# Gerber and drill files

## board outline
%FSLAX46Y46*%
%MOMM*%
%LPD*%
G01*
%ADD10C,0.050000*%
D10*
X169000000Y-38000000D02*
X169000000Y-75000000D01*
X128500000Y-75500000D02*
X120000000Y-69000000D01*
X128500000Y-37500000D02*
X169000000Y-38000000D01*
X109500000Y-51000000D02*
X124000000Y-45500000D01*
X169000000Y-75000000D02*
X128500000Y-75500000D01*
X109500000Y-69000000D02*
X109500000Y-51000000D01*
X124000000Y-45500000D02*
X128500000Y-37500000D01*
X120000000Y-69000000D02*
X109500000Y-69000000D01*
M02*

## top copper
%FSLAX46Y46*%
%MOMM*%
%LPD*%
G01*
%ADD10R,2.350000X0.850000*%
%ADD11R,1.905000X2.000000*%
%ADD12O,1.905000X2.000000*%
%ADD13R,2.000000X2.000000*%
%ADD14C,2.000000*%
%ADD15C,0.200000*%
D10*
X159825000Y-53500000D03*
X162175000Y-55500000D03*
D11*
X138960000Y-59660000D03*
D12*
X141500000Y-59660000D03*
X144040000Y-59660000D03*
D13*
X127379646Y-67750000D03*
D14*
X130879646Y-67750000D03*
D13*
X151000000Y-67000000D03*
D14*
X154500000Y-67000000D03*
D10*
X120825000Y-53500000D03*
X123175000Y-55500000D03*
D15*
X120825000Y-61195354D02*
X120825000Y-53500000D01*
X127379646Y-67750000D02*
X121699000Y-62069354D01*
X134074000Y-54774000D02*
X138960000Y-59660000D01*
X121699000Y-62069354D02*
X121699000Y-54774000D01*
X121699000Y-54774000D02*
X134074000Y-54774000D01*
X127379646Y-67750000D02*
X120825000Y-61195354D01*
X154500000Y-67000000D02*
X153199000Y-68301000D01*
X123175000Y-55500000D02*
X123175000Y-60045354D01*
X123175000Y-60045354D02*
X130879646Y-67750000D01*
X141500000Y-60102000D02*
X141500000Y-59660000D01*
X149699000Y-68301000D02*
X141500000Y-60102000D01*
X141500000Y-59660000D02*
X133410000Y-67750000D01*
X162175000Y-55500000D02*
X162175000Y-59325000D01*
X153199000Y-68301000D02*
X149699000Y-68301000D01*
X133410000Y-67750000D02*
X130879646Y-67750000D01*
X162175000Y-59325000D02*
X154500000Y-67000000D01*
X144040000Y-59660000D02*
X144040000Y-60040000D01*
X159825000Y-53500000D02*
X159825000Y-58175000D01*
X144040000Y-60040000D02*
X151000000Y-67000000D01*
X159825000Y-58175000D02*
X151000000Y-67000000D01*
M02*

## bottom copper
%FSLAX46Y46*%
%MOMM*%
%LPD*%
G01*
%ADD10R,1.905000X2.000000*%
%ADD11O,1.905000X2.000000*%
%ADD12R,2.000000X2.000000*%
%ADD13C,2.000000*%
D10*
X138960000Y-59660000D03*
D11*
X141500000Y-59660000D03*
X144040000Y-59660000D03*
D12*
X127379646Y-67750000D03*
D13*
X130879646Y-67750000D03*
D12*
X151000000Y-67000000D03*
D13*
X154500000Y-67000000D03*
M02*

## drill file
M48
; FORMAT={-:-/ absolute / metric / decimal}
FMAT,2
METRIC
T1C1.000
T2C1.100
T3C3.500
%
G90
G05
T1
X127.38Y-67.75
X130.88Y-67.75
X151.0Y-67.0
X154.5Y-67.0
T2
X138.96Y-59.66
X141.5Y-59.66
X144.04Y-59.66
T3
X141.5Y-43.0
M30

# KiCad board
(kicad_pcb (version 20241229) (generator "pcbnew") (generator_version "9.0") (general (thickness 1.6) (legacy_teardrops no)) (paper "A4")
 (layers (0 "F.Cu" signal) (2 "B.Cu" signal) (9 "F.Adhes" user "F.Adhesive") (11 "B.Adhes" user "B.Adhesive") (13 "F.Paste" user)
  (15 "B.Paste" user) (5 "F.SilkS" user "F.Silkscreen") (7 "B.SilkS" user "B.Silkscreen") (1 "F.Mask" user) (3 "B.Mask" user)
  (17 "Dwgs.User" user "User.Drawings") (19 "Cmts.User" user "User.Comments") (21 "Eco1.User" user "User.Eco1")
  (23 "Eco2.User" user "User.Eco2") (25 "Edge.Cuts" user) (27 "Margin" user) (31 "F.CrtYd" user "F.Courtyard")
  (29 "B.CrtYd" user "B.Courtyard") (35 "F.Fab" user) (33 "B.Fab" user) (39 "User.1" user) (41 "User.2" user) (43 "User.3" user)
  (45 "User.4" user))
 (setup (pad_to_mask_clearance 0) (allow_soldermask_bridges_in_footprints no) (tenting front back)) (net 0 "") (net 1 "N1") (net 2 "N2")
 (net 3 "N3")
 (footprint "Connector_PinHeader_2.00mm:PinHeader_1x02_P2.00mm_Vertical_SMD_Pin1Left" (layer "F.Cu") (at 161 54.5)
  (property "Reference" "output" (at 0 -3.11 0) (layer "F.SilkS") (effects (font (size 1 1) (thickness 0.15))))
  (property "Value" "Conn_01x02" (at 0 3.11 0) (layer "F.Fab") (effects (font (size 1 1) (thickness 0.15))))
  (pad "1" smd rect (at -1.175 -1) (size 2.35 0.85) (layers "F.Cu" "F.Mask" "F.Paste") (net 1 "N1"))
  (pad "2" smd rect (at 1.175 1) (size 2.35 0.85) (layers "F.Cu" "F.Mask" "F.Paste") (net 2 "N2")))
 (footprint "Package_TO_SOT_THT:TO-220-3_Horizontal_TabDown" (layer "F.Cu") (at 138.96 59.66)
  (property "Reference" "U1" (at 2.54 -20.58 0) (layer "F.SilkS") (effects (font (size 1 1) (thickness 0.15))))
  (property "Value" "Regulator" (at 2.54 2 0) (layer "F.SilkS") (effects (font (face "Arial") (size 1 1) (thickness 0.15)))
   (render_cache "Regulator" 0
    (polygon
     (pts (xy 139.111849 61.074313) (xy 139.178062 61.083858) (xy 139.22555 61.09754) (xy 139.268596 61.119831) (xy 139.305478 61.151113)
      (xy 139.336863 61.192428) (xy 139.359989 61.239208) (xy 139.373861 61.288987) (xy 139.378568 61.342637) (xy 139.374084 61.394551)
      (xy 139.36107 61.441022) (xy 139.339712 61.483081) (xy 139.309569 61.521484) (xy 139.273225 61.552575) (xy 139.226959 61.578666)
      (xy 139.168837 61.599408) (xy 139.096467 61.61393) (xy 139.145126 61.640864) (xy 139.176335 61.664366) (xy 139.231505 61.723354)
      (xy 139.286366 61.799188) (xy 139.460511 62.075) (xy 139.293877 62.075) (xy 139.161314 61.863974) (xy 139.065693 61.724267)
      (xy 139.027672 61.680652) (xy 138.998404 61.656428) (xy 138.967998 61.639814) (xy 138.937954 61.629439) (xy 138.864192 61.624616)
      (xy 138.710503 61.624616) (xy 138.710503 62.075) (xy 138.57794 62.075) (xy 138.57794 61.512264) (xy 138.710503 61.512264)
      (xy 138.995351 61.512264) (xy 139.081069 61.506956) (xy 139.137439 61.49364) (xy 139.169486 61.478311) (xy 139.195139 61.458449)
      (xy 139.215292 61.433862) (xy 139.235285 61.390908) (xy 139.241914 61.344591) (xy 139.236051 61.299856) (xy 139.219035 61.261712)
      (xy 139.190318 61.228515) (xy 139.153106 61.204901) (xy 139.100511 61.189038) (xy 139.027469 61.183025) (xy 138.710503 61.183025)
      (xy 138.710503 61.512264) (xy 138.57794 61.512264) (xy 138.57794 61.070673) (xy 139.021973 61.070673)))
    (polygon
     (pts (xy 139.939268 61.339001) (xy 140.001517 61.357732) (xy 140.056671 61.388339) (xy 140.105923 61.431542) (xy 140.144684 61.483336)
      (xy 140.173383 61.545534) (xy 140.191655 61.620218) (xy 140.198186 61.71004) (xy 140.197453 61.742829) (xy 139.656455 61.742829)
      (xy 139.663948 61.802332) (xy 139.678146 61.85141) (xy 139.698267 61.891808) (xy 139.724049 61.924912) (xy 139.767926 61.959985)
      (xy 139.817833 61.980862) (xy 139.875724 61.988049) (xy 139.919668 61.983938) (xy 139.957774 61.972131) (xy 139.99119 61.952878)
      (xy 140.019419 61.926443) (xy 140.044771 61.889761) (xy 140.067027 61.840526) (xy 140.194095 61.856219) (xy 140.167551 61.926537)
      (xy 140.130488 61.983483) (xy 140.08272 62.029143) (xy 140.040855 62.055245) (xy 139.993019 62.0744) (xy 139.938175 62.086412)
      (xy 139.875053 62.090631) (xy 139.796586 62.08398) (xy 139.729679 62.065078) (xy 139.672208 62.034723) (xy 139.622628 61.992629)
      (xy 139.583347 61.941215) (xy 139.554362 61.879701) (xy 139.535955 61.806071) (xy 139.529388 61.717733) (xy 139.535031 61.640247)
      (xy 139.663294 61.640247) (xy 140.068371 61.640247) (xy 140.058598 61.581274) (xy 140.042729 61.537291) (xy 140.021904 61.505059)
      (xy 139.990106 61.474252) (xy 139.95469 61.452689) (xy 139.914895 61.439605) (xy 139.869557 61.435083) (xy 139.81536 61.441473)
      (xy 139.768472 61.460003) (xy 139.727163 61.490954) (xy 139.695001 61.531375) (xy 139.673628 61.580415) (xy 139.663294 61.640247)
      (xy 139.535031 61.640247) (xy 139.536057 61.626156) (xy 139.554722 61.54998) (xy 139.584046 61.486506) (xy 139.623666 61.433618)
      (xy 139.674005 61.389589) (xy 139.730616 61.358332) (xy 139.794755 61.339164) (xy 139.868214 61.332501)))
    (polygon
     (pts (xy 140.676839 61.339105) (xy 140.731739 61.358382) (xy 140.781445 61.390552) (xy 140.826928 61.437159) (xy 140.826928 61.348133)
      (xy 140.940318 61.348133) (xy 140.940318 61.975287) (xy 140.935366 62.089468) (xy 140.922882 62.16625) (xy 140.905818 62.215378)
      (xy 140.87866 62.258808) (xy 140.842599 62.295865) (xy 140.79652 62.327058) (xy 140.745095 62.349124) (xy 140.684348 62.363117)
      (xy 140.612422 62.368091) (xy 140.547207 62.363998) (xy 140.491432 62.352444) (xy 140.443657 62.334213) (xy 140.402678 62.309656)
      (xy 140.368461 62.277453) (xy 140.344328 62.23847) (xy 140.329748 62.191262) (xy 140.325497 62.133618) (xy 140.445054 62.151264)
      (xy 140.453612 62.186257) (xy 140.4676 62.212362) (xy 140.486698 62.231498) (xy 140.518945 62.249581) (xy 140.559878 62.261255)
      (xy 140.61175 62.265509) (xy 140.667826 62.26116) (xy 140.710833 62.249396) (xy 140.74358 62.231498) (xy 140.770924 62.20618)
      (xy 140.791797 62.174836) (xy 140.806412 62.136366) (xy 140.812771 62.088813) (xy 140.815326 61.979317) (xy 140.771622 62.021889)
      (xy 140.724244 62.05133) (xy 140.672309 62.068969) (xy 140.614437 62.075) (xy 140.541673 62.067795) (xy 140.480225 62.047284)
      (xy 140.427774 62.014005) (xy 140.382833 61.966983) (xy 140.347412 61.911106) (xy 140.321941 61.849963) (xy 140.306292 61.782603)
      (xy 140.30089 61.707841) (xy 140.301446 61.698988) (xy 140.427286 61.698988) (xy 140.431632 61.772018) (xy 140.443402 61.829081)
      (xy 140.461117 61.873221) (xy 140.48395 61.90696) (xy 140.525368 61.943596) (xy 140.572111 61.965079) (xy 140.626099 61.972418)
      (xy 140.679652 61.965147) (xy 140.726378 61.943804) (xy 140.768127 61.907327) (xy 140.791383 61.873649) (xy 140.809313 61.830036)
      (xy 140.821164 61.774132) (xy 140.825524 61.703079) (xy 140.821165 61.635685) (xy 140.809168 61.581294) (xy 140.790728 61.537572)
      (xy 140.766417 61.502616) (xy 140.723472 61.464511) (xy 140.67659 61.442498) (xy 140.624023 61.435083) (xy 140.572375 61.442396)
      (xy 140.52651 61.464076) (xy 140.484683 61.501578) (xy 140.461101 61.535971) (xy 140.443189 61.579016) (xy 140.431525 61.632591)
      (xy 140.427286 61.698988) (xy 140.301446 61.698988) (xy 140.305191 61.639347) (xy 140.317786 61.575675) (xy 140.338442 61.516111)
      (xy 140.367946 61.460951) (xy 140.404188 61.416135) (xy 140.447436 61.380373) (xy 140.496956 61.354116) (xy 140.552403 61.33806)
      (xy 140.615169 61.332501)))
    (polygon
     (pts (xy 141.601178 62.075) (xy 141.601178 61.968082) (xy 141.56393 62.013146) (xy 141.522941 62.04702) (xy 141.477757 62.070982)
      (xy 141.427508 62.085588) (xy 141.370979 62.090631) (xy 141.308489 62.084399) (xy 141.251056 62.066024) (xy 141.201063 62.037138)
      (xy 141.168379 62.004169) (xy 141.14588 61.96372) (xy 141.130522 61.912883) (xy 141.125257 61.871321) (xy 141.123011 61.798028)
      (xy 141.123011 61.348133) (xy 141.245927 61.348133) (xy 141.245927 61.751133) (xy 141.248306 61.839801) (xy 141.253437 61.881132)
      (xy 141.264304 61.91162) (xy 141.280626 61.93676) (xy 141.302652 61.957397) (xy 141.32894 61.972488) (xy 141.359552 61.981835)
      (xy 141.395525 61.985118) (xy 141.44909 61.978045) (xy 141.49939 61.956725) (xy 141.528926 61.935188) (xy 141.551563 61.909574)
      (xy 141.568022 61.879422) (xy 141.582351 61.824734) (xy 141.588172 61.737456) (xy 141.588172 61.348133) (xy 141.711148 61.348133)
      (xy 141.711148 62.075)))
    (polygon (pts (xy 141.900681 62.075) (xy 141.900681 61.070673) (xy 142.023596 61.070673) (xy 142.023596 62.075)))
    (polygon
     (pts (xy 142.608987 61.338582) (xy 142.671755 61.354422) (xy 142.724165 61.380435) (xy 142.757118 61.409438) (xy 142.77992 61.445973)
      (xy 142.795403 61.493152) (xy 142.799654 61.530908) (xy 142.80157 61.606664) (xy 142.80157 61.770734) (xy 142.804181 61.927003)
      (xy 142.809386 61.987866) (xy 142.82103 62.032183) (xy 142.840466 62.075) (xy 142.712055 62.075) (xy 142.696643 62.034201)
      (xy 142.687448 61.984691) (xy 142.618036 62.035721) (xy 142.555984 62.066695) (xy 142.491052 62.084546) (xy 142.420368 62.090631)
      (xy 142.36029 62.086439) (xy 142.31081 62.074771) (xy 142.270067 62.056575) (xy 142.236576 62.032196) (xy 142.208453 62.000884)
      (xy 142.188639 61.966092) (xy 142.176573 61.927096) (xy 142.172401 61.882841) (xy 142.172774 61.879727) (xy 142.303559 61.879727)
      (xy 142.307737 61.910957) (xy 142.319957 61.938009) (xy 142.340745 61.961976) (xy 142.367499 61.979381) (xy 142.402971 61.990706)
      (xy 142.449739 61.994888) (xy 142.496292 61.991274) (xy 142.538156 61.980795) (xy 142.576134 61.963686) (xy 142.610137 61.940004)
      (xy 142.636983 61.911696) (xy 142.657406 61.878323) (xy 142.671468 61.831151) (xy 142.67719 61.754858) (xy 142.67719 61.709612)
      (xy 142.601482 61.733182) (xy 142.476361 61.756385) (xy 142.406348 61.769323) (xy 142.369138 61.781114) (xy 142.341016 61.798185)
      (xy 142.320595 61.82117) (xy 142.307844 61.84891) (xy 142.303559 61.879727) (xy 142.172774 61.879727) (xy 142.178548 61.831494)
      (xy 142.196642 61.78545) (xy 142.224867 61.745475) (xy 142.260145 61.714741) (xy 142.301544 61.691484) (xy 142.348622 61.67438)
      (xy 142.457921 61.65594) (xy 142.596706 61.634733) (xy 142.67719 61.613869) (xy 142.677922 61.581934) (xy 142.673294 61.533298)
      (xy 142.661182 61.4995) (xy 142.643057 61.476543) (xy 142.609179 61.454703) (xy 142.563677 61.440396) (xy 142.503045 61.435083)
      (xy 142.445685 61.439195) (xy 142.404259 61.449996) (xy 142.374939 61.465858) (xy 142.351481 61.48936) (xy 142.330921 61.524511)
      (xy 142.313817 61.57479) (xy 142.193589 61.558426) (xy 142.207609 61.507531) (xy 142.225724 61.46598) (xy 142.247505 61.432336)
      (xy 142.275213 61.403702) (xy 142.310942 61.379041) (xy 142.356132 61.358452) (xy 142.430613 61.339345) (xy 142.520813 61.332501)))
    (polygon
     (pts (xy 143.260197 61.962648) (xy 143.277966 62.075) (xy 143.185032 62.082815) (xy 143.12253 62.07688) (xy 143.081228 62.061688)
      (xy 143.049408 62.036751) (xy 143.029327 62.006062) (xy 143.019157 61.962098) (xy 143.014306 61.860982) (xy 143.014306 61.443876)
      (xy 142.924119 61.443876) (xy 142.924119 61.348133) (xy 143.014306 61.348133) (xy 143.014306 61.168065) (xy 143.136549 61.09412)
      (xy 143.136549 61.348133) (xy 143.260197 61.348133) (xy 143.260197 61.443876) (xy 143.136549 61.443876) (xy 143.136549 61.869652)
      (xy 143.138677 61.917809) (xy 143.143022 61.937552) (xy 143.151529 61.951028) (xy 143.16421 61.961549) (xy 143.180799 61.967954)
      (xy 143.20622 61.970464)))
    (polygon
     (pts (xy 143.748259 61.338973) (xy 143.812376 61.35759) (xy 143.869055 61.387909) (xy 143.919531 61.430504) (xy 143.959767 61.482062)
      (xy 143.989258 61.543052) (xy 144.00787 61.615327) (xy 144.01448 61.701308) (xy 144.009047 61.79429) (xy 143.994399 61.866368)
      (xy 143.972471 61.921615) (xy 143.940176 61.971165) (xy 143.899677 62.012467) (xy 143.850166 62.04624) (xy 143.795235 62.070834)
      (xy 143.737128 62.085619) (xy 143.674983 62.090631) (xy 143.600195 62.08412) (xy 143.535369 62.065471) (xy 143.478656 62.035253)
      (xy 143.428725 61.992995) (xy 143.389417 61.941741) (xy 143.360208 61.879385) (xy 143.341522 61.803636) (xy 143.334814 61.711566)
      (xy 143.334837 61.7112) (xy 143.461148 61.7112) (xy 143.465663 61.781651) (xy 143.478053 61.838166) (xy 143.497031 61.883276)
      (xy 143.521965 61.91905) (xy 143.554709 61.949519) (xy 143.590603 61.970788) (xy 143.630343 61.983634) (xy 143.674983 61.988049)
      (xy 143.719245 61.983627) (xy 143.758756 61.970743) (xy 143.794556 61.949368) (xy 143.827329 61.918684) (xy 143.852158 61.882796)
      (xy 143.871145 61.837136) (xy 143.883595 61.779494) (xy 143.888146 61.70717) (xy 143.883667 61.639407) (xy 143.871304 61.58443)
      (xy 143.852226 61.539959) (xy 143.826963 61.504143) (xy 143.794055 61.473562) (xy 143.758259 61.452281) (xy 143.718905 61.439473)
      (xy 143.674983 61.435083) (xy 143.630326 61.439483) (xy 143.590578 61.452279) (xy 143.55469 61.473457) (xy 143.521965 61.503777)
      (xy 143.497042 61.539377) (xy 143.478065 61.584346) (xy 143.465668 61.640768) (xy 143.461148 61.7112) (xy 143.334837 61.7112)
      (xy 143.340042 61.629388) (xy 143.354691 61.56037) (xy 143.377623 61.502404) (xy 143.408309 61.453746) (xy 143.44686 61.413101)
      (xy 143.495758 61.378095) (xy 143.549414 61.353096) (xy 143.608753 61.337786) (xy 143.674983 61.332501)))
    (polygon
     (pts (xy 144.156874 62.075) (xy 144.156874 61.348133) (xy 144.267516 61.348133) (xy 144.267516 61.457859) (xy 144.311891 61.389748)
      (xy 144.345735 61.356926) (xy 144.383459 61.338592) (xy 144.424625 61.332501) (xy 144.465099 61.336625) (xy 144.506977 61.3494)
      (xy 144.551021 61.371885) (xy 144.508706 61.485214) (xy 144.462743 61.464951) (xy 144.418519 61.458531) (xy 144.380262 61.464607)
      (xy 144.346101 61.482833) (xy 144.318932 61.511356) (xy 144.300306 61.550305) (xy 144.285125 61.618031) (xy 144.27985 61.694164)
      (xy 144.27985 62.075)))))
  (pad "" np_thru_hole circle (at 2.54 -16.66) (size 3.5 3.5) (drill 3.5) (layers "*.Cu" "*.Mask"))
  (pad "1" thru_hole rect (at 0 0) (size 1.905 2) (drill 1.1) (layers "*.Cu" "*.Mask") (remove_unused_layers no) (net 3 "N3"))
  (pad "2" thru_hole oval (at 2.54 0) (size 1.905 2) (drill 1.1) (layers "*.Cu" "*.Mask") (remove_unused_layers no) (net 2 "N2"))
  (pad "3" thru_hole oval (at 5.08 0) (size 1.905 2) (drill 1.1) (layers "*.Cu" "*.Mask") (remove_unused_layers no) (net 1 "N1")))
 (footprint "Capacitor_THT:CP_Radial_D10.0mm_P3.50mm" (layer "F.Cu") (at 127.379646 67.75)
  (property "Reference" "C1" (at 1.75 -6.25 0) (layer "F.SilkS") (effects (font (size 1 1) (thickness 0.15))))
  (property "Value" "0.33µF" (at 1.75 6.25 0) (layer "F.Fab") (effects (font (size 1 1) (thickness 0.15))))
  (pad "1" thru_hole rect (at 0 0) (size 2 2) (drill 1) (layers "*.Cu" "*.Mask") (remove_unused_layers no) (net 3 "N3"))
  (pad "2" thru_hole circle (at 3.5 0) (size 2 2) (drill 1) (layers "*.Cu" "*.Mask") (remove_unused_layers no) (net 2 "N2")))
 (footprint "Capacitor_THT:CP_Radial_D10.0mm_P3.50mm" (layer "F.Cu") (at 151 67)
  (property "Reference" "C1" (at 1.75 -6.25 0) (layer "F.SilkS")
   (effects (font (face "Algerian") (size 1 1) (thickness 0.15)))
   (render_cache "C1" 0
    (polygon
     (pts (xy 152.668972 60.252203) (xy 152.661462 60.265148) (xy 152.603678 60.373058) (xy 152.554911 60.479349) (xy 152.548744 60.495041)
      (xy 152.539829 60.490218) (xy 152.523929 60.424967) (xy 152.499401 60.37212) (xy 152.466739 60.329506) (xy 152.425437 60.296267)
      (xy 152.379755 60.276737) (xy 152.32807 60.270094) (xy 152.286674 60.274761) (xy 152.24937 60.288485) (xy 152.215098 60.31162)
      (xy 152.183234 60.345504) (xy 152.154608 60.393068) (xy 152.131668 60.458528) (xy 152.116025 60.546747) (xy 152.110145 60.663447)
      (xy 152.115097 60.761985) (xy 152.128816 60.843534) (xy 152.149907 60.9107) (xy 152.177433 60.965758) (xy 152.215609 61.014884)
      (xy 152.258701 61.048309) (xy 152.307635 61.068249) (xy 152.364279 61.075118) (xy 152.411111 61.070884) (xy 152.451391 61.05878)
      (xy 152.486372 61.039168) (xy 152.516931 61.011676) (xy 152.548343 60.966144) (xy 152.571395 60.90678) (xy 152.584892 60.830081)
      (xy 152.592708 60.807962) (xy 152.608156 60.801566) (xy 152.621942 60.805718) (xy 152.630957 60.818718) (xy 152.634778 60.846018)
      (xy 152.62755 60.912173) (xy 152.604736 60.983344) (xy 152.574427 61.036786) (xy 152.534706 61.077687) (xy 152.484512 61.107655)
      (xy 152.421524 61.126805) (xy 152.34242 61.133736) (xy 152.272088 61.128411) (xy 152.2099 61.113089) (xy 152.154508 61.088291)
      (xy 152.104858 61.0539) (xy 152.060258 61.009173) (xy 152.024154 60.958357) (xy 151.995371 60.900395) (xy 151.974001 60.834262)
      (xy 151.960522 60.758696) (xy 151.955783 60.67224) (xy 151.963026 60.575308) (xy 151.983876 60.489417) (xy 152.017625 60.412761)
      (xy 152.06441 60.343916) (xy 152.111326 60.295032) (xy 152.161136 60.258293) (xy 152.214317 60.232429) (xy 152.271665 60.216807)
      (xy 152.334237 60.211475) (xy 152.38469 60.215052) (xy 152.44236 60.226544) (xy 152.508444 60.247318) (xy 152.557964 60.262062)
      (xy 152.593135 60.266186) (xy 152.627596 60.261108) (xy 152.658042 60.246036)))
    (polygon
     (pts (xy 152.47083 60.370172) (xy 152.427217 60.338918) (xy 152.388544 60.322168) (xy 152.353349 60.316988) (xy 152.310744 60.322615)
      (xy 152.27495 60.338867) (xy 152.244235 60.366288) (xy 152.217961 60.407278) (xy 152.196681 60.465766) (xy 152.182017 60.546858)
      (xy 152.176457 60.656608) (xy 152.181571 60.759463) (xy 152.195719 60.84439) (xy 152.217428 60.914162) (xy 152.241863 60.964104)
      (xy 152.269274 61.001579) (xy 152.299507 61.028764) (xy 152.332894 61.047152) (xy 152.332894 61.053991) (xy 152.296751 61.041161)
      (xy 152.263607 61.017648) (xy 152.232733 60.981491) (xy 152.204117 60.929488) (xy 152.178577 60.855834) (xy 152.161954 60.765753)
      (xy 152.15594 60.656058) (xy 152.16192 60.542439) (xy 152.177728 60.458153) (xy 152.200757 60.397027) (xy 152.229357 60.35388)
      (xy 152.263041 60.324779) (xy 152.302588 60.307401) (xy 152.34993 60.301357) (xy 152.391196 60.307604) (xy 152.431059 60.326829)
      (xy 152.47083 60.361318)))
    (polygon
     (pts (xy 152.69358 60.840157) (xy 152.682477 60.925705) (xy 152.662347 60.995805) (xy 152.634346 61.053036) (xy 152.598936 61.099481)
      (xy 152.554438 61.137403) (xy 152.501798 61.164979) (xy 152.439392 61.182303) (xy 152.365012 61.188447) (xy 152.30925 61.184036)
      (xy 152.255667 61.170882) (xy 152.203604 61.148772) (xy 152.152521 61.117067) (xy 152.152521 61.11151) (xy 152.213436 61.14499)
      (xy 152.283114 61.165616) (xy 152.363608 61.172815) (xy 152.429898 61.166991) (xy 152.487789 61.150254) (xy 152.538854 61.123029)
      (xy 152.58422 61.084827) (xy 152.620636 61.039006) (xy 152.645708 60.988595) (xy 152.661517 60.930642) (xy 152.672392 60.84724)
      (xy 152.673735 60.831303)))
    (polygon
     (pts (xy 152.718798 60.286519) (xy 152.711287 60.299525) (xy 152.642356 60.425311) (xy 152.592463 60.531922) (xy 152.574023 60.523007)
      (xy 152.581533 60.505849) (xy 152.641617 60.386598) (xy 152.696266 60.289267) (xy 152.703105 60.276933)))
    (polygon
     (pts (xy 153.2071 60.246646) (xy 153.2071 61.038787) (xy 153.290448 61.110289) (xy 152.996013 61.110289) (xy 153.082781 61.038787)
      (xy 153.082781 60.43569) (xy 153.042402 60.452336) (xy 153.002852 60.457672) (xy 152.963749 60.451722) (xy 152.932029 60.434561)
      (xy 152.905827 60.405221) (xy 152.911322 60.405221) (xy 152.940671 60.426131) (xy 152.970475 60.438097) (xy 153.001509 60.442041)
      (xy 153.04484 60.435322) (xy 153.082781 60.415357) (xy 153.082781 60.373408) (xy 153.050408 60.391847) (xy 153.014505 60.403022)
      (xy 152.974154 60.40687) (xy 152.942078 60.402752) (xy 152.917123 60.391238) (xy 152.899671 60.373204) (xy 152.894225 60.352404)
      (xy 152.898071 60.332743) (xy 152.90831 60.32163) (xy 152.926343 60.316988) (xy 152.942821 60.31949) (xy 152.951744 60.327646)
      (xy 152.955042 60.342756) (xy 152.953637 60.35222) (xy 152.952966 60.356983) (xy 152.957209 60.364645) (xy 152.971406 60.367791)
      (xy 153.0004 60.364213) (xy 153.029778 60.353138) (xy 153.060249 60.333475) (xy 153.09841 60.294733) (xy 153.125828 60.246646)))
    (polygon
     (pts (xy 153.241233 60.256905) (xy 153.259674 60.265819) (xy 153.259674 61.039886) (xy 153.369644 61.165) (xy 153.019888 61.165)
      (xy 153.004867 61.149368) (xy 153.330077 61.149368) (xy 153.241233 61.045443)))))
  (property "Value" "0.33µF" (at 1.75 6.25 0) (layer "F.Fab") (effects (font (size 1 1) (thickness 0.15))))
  (pad "1" thru_hole rect (at 0 0) (size 2 2) (drill 1) (layers "*.Cu" "*.Mask") (remove_unused_layers no) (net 1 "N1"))
  (pad "2" thru_hole circle (at 3.5 0) (size 2 2) (drill 1) (layers "*.Cu" "*.Mask") (remove_unused_layers no) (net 2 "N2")))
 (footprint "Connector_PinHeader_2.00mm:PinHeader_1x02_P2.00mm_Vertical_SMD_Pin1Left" (layer "F.Cu") (at 122 54.5)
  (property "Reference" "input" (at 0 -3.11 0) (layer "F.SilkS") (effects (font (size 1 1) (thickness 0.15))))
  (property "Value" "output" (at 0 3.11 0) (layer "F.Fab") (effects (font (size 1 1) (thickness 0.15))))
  (pad "1" smd rect (at -1.175 -1) (size 2.35 0.85) (layers "F.Cu" "F.Mask" "F.Paste") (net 3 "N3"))
  (pad "2" smd rect (at 1.175 1) (size 2.35 0.85) (layers "F.Cu" "F.Mask" "F.Paste") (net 2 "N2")))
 (gr_line (start 169 38) (end 169 75) (stroke (width 0.05) (type default)) (layer "Edge.Cuts"))
 (gr_line (start 128.5 75.5) (end 120 69) (stroke (width 0.05) (type default)) (layer "Edge.Cuts"))
 (gr_line (start 128.5 37.5) (end 169 38) (stroke (width 0.05) (type default)) (layer "Edge.Cuts"))
 (gr_line (start 109.5 51) (end 124 45.5) (stroke (width 0.05) (type default)) (layer "Edge.Cuts"))
 (gr_line (start 169 75) (end 128.5 75.5) (stroke (width 0.05) (type default)) (layer "Edge.Cuts"))
 (gr_line (start 109.5 69) (end 109.5 51) (stroke (width 0.05) (type default)) (layer "Edge.Cuts"))
 (gr_line (start 124 45.5) (end 128.5 37.5) (stroke (width 0.05) (type default)) (layer "Edge.Cuts"))
 (gr_line (start 120 69) (end 109.5 69) (stroke (width 0.05) (type default)) (layer "Edge.Cuts"))
 (segment (start 120.825 61.195354) (end 120.825 53.5) (width 0.2) (layer "F.Cu") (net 3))
 (segment (start 127.379646 67.75) (end 121.699 62.069354) (width 0.2) (layer "F.Cu") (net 3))
 (segment (start 134.074 54.774) (end 138.96 59.66) (width 0.2) (layer "F.Cu") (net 3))
 (segment (start 121.699 62.069354) (end 121.699 54.774) (width 0.2) (layer "F.Cu") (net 3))
 (segment (start 121.699 54.774) (end 134.074 54.774) (width 0.2) (layer "F.Cu") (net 3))
 (segment (start 127.379646 67.75) (end 120.825 61.195354) (width 0.2) (layer "F.Cu") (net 3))
 (segment (start 154.5 67) (end 153.199 68.301) (width 0.2) (layer "F.Cu") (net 2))
 (segment (start 123.175 55.5) (end 123.175 60.045354) (width 0.2) (layer "F.Cu") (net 2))
 (segment (start 123.175 60.045354) (end 130.879646 67.75) (width 0.2) (layer "F.Cu") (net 2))
 (segment (start 141.5 60.102) (end 141.5 59.66) (width 0.2) (layer "F.Cu") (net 2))
 (segment (start 149.699 68.301) (end 141.5 60.102) (width 0.2) (layer "F.Cu") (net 2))
 (segment (start 141.5 59.66) (end 133.41 67.75) (width 0.2) (layer "F.Cu") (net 2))
 (segment (start 162.175 55.5) (end 162.175 59.325) (width 0.2) (layer "F.Cu") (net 2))
 (segment (start 153.199 68.301) (end 149.699 68.301) (width 0.2) (layer "F.Cu") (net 2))
 (segment (start 133.41 67.75) (end 130.879646 67.75) (width 0.2) (layer "F.Cu") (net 2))
 (segment (start 162.175 59.325) (end 154.5 67) (width 0.2) (layer "F.Cu") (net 2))
 (segment (start 144.04 59.66) (end 144.04 60.04) (width 0.2) (layer "F.Cu") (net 1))
 (segment (start 159.825 53.5) (end 159.825 58.175) (width 0.2) (layer "F.Cu") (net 1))
 (segment (start 144.04 60.04) (end 151 67) (width 0.2) (layer "F.Cu") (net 1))
 (segment (start 159.825 58.175) (end 151 67) (width 0.2) (layer "F.Cu") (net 1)))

